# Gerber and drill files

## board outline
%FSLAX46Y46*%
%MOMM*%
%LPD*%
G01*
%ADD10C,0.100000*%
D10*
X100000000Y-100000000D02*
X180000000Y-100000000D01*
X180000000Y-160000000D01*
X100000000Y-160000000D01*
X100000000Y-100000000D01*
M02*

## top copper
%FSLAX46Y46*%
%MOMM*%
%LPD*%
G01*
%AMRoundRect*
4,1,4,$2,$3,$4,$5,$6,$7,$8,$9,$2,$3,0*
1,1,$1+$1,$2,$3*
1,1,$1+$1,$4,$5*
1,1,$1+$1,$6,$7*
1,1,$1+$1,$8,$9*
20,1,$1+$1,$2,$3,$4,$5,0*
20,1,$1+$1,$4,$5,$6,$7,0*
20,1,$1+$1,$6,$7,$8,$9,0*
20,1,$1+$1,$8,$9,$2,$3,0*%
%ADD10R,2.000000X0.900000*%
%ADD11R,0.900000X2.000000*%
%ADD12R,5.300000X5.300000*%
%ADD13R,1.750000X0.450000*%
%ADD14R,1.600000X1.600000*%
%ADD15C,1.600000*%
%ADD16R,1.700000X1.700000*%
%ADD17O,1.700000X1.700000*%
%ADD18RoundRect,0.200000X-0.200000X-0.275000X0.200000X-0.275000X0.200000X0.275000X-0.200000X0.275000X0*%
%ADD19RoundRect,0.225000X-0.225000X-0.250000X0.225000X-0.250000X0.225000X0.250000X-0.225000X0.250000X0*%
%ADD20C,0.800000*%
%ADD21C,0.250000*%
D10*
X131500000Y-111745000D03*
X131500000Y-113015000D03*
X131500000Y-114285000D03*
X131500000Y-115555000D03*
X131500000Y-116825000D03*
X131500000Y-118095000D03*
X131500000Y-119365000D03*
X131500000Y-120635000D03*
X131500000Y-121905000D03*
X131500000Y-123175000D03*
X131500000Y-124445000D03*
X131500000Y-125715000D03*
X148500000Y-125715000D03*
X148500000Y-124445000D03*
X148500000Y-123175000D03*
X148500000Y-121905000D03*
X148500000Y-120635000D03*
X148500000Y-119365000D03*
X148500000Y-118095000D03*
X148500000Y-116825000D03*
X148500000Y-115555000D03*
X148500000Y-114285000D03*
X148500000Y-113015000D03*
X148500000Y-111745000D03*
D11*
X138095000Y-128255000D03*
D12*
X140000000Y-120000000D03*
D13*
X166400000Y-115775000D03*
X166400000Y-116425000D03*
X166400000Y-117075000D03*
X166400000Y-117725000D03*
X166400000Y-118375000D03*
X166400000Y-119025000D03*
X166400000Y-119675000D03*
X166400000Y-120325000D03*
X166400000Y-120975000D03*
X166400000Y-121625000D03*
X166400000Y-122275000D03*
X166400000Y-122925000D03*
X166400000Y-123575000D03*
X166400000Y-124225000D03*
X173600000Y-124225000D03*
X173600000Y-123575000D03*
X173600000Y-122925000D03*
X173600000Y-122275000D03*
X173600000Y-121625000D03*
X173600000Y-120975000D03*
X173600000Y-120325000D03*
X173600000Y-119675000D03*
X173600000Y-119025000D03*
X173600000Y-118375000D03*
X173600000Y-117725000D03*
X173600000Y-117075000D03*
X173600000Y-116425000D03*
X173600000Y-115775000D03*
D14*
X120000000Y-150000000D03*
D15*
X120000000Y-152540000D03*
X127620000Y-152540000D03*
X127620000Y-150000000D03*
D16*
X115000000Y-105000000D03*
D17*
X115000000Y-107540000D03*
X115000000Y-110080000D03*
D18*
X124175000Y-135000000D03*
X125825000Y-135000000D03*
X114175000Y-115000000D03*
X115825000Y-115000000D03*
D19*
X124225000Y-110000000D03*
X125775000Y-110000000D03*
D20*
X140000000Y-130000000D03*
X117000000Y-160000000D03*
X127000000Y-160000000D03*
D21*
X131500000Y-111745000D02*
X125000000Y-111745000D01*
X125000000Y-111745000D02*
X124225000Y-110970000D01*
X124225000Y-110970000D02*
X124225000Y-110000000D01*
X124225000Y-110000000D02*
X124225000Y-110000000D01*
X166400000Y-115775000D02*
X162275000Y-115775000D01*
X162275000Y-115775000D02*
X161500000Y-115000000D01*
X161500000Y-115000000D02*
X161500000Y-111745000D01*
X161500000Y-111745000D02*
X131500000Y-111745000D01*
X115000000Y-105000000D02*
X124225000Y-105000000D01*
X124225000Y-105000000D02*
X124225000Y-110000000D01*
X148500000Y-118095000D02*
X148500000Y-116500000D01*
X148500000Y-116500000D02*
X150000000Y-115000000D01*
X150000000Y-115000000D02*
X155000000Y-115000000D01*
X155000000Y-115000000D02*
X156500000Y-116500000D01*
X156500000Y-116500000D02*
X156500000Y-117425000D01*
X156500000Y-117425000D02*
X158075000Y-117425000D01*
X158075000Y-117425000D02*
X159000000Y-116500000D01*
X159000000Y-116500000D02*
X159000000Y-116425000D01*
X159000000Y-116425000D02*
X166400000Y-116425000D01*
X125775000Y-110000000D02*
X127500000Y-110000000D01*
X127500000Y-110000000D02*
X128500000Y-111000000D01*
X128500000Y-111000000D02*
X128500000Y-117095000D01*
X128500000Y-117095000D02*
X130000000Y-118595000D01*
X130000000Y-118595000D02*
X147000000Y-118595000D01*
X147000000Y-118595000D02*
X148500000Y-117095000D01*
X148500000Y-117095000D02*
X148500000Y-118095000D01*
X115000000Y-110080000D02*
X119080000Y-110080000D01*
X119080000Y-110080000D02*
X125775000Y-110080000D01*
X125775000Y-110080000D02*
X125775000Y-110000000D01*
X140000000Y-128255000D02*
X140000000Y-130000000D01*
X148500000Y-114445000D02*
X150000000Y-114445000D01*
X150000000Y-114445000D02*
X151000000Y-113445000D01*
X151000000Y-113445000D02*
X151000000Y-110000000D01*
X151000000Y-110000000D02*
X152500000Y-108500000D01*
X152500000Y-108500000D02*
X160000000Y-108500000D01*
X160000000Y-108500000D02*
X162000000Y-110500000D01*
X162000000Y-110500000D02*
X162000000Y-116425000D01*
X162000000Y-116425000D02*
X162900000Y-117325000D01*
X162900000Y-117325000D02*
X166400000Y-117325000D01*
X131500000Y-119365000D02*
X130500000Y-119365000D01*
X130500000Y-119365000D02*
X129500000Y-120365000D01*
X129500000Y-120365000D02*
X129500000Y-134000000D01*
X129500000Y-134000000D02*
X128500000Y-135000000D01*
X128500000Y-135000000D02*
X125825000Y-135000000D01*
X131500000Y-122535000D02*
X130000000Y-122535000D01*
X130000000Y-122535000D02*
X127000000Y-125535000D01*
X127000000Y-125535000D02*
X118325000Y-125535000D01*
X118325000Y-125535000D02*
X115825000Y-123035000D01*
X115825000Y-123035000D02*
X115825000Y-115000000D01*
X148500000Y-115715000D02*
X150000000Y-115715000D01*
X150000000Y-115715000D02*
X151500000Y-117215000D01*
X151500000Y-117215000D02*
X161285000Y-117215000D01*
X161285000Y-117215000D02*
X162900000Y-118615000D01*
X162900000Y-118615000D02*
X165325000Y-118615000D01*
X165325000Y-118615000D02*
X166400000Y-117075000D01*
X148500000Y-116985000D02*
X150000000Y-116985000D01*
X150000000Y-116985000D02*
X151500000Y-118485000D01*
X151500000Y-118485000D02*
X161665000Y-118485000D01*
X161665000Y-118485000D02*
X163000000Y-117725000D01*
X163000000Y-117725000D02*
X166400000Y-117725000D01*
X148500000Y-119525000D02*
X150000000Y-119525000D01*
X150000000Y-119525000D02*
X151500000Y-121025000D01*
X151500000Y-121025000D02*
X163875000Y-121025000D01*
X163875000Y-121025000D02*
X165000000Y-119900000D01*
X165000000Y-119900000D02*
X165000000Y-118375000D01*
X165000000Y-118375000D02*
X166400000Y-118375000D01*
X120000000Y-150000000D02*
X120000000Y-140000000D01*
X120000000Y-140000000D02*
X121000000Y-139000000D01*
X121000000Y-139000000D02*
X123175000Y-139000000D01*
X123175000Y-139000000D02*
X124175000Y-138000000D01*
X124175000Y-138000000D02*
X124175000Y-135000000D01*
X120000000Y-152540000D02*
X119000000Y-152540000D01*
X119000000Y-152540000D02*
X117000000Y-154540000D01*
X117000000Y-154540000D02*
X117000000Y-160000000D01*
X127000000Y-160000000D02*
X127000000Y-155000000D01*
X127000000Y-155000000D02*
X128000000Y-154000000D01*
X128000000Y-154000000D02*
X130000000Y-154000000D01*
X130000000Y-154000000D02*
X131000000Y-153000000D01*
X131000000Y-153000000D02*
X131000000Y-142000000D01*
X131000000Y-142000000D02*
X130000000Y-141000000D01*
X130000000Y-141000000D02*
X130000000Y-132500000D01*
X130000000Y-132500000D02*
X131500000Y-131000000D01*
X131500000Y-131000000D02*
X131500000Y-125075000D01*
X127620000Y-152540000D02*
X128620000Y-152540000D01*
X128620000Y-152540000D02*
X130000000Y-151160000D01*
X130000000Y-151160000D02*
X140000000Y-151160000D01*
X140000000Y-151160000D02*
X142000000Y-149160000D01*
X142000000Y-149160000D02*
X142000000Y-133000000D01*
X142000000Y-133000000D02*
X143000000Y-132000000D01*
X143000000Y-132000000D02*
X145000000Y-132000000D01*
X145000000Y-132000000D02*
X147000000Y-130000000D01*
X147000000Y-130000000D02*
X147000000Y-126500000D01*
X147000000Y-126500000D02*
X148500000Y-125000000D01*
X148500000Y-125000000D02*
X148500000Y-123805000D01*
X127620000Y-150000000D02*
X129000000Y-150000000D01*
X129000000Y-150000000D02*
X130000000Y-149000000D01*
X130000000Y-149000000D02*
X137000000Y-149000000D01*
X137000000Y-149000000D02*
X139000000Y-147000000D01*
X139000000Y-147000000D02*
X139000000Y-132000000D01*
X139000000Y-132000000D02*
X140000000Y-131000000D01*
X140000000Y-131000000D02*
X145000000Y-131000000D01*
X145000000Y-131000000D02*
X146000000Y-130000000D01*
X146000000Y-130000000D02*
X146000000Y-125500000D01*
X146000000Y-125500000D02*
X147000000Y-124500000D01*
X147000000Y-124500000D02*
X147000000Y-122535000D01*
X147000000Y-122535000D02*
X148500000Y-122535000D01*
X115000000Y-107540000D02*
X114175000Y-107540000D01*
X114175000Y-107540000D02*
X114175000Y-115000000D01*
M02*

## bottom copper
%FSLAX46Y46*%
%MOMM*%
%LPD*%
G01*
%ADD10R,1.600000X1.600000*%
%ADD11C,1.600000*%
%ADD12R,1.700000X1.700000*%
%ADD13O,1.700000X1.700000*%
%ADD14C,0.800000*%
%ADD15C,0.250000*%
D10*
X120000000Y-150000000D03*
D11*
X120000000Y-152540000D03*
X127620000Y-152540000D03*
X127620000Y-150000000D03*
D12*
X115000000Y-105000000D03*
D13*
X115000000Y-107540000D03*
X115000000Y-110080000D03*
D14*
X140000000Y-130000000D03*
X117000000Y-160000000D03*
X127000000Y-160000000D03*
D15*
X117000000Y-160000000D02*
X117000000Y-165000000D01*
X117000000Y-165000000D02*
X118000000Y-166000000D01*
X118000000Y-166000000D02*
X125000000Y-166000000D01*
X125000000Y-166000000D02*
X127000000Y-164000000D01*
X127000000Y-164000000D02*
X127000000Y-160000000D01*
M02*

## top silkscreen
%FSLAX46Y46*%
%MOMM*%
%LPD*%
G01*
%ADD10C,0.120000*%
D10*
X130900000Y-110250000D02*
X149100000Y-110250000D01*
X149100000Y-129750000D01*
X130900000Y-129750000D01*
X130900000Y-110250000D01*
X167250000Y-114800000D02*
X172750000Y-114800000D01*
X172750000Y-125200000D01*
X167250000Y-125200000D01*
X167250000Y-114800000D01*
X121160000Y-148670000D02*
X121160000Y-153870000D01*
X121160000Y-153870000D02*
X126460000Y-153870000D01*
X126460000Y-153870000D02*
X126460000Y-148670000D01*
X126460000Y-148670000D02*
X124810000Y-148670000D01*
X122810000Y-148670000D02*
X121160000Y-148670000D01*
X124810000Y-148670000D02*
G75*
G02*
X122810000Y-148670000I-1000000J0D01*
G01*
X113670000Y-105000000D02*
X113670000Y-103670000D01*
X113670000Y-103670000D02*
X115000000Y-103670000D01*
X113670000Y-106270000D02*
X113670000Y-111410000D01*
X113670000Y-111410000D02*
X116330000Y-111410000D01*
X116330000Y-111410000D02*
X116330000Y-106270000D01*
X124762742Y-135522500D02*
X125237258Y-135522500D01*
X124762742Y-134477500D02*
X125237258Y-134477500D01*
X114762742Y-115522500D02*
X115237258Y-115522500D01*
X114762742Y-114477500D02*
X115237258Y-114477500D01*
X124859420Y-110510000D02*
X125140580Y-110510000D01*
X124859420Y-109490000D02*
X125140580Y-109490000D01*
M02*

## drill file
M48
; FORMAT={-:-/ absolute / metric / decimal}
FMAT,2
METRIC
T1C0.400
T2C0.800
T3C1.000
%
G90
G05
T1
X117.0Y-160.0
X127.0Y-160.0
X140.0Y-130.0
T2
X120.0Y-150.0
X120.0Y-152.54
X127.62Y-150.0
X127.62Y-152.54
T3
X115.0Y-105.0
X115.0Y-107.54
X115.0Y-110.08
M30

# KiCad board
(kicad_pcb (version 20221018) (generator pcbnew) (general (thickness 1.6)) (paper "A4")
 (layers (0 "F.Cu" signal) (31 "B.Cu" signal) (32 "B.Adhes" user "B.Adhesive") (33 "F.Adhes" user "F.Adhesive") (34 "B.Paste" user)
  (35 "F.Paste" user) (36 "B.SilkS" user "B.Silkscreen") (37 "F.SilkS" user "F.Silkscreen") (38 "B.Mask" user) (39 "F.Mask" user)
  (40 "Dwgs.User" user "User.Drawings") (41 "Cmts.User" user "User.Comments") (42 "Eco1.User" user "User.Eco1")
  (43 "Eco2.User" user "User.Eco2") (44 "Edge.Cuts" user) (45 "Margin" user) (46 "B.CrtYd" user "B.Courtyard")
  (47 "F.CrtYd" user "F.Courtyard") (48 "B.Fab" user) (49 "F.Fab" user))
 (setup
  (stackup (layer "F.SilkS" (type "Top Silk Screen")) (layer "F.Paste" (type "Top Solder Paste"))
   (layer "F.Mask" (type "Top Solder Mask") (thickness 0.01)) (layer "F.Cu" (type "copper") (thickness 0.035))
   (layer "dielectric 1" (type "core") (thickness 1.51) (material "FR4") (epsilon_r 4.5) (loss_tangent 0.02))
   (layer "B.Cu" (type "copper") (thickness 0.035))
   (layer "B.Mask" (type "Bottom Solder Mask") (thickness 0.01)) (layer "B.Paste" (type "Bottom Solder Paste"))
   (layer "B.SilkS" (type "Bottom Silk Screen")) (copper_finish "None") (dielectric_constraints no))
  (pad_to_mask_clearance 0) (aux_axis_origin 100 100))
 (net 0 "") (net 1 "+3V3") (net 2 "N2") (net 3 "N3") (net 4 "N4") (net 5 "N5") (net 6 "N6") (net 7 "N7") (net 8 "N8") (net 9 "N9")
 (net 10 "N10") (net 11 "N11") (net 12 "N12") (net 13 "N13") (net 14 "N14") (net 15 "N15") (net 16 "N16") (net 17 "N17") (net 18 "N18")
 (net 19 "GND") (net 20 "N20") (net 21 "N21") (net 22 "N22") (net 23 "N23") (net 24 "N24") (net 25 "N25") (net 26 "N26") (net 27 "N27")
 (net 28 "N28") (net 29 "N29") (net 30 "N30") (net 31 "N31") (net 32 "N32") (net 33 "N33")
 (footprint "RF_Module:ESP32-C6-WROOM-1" (layer "F.Cu") (at 140 120 0)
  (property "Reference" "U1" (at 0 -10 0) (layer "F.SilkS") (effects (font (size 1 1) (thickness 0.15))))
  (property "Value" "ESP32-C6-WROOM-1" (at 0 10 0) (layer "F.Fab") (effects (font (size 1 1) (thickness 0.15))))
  (fp_rect (start -9.1 -9.75) (end 9.1 9.75) (layer "F.SilkS") (width 0.12) (fill none))
  (pad "1" smd rect (at -8.5 -8.255) (size 2 0.9) (layers "F.Cu" "F.Paste" "F.Mask") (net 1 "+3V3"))
  (pad "2" smd rect (at -8.5 -6.985) (size 2 0.9) (layers "F.Cu" "F.Paste" "F.Mask") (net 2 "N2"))
  (pad "3" smd rect (at -8.5 -5.715) (size 2 0.9) (layers "F.Cu" "F.Paste" "F.Mask") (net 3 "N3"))
  (pad "4" smd rect (at -8.5 -4.445) (size 2 0.9) (layers "F.Cu" "F.Paste" "F.Mask") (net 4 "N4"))
  (pad "5" smd rect (at -8.5 -3.175) (size 2 0.9) (layers "F.Cu" "F.Paste" "F.Mask") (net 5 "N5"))
  (pad "6" smd rect (at -8.5 -1.905) (size 2 0.9) (layers "F.Cu" "F.Paste" "F.Mask") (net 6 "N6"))
  (pad "7" smd rect (at -8.5 -0.635) (size 2 0.9) (layers "F.Cu" "F.Paste" "F.Mask") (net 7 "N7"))
  (pad "8" smd rect (at -8.5 0.635) (size 2 0.9) (layers "F.Cu" "F.Paste" "F.Mask") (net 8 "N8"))
  (pad "9" smd rect (at -8.5 1.905) (size 2 0.9) (layers "F.Cu" "F.Paste" "F.Mask") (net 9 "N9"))
  (pad "10" smd rect (at -8.5 3.175) (size 2 0.9) (layers "F.Cu" "F.Paste" "F.Mask") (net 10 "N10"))
  (pad "11" smd rect (at -8.5 4.445) (size 2 0.9) (layers "F.Cu" "F.Paste" "F.Mask") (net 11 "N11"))
  (pad "12" smd rect (at -8.5 5.715) (size 2 0.9) (layers "F.Cu" "F.Paste" "F.Mask") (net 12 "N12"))
  (pad "13" smd rect (at 8.5 5.715) (size 2 0.9) (layers "F.Cu" "F.Paste" "F.Mask") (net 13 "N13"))
  (pad "14" smd rect (at 8.5 4.445) (size 2 0.9) (layers "F.Cu" "F.Paste" "F.Mask") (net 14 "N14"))
  (pad "15" smd rect (at 8.5 3.175) (size 2 0.9) (layers "F.Cu" "F.Paste" "F.Mask") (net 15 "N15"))
  (pad "16" smd rect (at 8.5 1.905) (size 2 0.9) (layers "F.Cu" "F.Paste" "F.Mask") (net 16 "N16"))
  (pad "17" smd rect (at 8.5 0.635) (size 2 0.9) (layers "F.Cu" "F.Paste" "F.Mask") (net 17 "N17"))
  (pad "18" smd rect (at 8.5 -0.635) (size 2 0.9) (layers "F.Cu" "F.Paste" "F.Mask") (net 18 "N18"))
  (pad "19" smd rect (at 8.5 -1.905) (size 2 0.9) (layers "F.Cu" "F.Paste" "F.Mask") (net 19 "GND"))
  (pad "20" smd rect (at 8.5 -3.175) (size 2 0.9) (layers "F.Cu" "F.Paste" "F.Mask") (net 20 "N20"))
  (pad "21" smd rect (at 8.5 -4.445) (size 2 0.9) (layers "F.Cu" "F.Paste" "F.Mask") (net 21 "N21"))
  (pad "22" smd rect (at 8.5 -5.715) (size 2 0.9) (layers "F.Cu" "F.Paste" "F.Mask") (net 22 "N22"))
  (pad "23" smd rect (at 8.5 -6.985) (size 2 0.9) (layers "F.Cu" "F.Paste" "F.Mask") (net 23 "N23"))
  (pad "24" smd rect (at 8.5 -8.255) (size 2 0.9) (layers "F.Cu" "F.Paste" "F.Mask") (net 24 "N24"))
  (pad "25" smd rect (at -1.905 8.255 90) (size 2 0.9) (layers "F.Cu" "F.Paste" "F.Mask") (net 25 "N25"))
  (pad "39" smd rect (at 0 0) (size 5.3 5.3) (layers "F.Cu" "F.Paste" "F.Mask") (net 19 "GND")))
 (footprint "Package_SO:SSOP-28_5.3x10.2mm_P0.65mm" (layer "F.Cu") (at 170 120 0)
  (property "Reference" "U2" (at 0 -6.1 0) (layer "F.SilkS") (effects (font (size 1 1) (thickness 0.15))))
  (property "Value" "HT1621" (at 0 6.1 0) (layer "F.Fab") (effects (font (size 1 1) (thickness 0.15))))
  (fp_rect (start -2.75 -5.2) (end 2.75 5.2) (layer "F.SilkS") (width 0.12) (fill none))
  (pad "1" smd rect (at -3.6 -4.225) (size 1.75 0.45) (layers "F.Cu" "F.Paste" "F.Mask") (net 1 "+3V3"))
  (pad "2" smd rect (at -3.6 -3.575) (size 1.75 0.45) (layers "F.Cu" "F.Paste" "F.Mask") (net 19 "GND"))
  (pad "3" smd rect (at -3.6 -2.925) (size 1.75 0.45) (layers "F.Cu" "F.Paste" "F.Mask") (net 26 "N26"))
  (pad "4" smd rect (at -3.6 -2.275) (size 1.75 0.45) (layers "F.Cu" "F.Paste" "F.Mask") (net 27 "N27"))
  (pad "5" smd rect (at -3.6 -1.625) (size 1.75 0.45) (layers "F.Cu" "F.Paste" "F.Mask") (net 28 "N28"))
  (pad "6" smd rect (at -3.6 -0.975) (size 1.75 0.45) (layers "F.Cu" "F.Paste" "F.Mask"))
  (pad "7" smd rect (at -3.6 -0.325) (size 1.75 0.45) (layers "F.Cu" "F.Paste" "F.Mask"))
  (pad "8" smd rect (at -3.6 0.325) (size 1.75 0.45) (layers "F.Cu" "F.Paste" "F.Mask"))
  (pad "9" smd rect (at -3.6 0.975) (size 1.75 0.45) (layers "F.Cu" "F.Paste" "F.Mask"))
  (pad "10" smd rect (at -3.6 1.625) (size 1.75 0.45) (layers "F.Cu" "F.Paste" "F.Mask"))
  (pad "11" smd rect (at -3.6 2.275) (size 1.75 0.45) (layers "F.Cu" "F.Paste" "F.Mask"))
  (pad "12" smd rect (at -3.6 2.925) (size 1.75 0.45) (layers "F.Cu" "F.Paste" "F.Mask"))
  (pad "13" smd rect (at -3.6 3.575) (size 1.75 0.45) (layers "F.Cu" "F.Paste" "F.Mask"))
  (pad "14" smd rect (at -3.6 4.225) (size 1.75 0.45) (layers "F.Cu" "F.Paste" "F.Mask"))
  (pad "15" smd rect (at 3.6 4.225) (size 1.75 0.45) (layers "F.Cu" "F.Paste" "F.Mask"))
  (pad "16" smd rect (at 3.6 3.575) (size 1.75 0.45) (layers "F.Cu" "F.Paste" "F.Mask"))
  (pad "17" smd rect (at 3.6 2.925) (size 1.75 0.45) (layers "F.Cu" "F.Paste" "F.Mask"))
  (pad "18" smd rect (at 3.6 2.275) (size 1.75 0.45) (layers "F.Cu" "F.Paste" "F.Mask"))
  (pad "19" smd rect (at 3.6 1.625) (size 1.75 0.45) (layers "F.Cu" "F.Paste" "F.Mask"))
  (pad "20" smd rect (at 3.6 0.975) (size 1.75 0.45) (layers "F.Cu" "F.Paste" "F.Mask"))
  (pad "21" smd rect (at 3.6 0.325) (size 1.75 0.45) (layers "F.Cu" "F.Paste" "F.Mask"))
  (pad "22" smd rect (at 3.6 -0.325) (size 1.75 0.45) (layers "F.Cu" "F.Paste" "F.Mask"))
  (pad "23" smd rect (at 3.6 -0.975) (size 1.75 0.45) (layers "F.Cu" "F.Paste" "F.Mask"))
  (pad "24" smd rect (at 3.6 -1.625) (size 1.75 0.45) (layers "F.Cu" "F.Paste" "F.Mask"))
  (pad "25" smd rect (at 3.6 -2.275) (size 1.75 0.45) (layers "F.Cu" "F.Paste" "F.Mask"))
  (pad "26" smd rect (at 3.6 -2.925) (size 1.75 0.45) (layers "F.Cu" "F.Paste" "F.Mask"))
  (pad "27" smd rect (at 3.6 -3.575) (size 1.75 0.45) (layers "F.Cu" "F.Paste" "F.Mask"))
  (pad "28" smd rect (at 3.6 -4.225) (size 1.75 0.45) (layers "F.Cu" "F.Paste" "F.Mask")))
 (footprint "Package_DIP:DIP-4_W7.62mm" (layer "F.Cu") (at 120 150 0)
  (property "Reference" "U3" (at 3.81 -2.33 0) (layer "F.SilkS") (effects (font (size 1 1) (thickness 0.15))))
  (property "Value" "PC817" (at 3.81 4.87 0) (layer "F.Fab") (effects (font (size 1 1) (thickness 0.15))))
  (fp_line (start 1.16 -1.33) (end 1.16 3.87) (layer "F.SilkS") (width 0.12))
  (fp_line (start 1.16 3.87) (end 6.46 3.87) (layer "F.SilkS") (width 0.12))
  (fp_line (start 6.46 3.87) (end 6.46 -1.33) (layer "F.SilkS") (width 0.12))
  (fp_line (start 6.46 -1.33) (end 4.81 -1.33) (layer "F.SilkS") (width 0.12))
  (fp_line (start 2.81 -1.33) (end 1.16 -1.33) (layer "F.SilkS") (width 0.12))
  (fp_arc (start 4.81 -1.33) (mid 3.81 -0.33) (end 2.81 -1.33) (layer "F.SilkS") (width 0.12))
  (pad "1" thru_hole rect (at 0 0) (size 1.6 1.6) (drill 0.8) (layers *.Cu *.Mask) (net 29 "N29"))
  (pad "2" thru_hole circle (at 0 2.54) (size 1.6 1.6) (drill 0.8) (layers *.Cu *.Mask) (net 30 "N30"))
  (pad "3" thru_hole circle (at 7.62 2.54) (size 1.6 1.6) (drill 0.8) (layers *.Cu *.Mask) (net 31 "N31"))
  (pad "4" thru_hole circle (at 7.62 0) (size 1.6 1.6) (drill 0.8) (layers *.Cu *.Mask) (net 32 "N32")))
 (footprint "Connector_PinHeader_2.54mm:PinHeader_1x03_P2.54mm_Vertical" (layer "F.Cu") (at 115 105 0)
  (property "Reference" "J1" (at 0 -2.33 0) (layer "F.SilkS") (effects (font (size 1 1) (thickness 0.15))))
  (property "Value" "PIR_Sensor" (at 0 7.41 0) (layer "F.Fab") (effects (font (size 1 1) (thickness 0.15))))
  (fp_line (start -1.33 0) (end -1.33 -1.33) (layer "F.SilkS") (width 0.12))
  (fp_line (start -1.33 -1.33) (end 0 -1.33) (layer "F.SilkS") (width 0.12))
  (fp_line (start -1.33 1.27) (end -1.33 6.41) (layer "F.SilkS") (width 0.12))
  (fp_line (start -1.33 6.41) (end 1.33 6.41) (layer "F.SilkS") (width 0.12))
  (fp_line (start 1.33 6.41) (end 1.33 1.27) (layer "F.SilkS") (width 0.12))
  (pad "1" thru_hole rect (at 0 0) (size 1.7 1.7) (drill 1) (layers *.Cu *.Mask) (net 1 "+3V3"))
  (pad "2" thru_hole oval (at 0 2.54) (size 1.7 1.7) (drill 1) (layers *.Cu *.Mask) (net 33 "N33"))
  (pad "3" thru_hole oval (at 0 5.08) (size 1.7 1.7) (drill 1) (layers *.Cu *.Mask) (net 19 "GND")))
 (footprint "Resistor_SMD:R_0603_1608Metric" (layer "F.Cu") (at 125 135 0)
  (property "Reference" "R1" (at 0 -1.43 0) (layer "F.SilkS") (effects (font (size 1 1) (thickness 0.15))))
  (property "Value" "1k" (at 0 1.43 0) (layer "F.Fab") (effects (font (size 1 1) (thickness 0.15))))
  (fp_line (start -0.237258 0.5225) (end 0.237258 0.5225) (layer "F.SilkS") (width 0.12))
  (fp_line (start -0.237258 -0.5225) (end 0.237258 -0.5225) (layer "F.SilkS") (width 0.12))
  (pad "1" smd roundrect (at -0.825 0) (size 0.8 0.95) (layers "F.Cu" "F.Paste" "F.Mask") (roundrect_rratio 0.25) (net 29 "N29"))
  (pad "2" smd roundrect (at 0.825 0) (size 0.8 0.95) (layers "F.Cu" "F.Paste" "F.Mask") (roundrect_rratio 0.25) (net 7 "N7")))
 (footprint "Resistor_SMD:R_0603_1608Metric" (layer "F.Cu") (at 115 115 0)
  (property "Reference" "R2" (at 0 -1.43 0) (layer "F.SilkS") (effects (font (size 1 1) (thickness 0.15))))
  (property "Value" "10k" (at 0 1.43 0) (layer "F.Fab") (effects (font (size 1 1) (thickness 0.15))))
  (fp_line (start -0.237258 0.5225) (end 0.237258 0.5225) (layer "F.SilkS") (width 0.12))
  (fp_line (start -0.237258 -0.5225) (end 0.237258 -0.5225) (layer "F.SilkS") (width 0.12))
  (pad "1" smd roundrect (at -0.825 0) (size 0.8 0.95) (layers "F.Cu" "F.Paste" "F.Mask") (roundrect_rratio 0.25) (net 33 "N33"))
  (pad "2" smd roundrect (at 0.825 0) (size 0.8 0.95) (layers "F.Cu" "F.Paste" "F.Mask") (roundrect_rratio 0.25) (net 9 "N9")))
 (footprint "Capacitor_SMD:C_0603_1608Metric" (layer "F.Cu") (at 125 110 0)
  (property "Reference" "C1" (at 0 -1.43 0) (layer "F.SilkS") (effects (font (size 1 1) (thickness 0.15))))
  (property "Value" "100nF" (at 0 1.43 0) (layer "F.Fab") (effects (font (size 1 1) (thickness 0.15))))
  (fp_line (start -0.14058 0.51) (end 0.14058 0.51) (layer "F.SilkS") (width 0.12))
  (fp_line (start -0.14058 -0.51) (end 0.14058 -0.51) (layer "F.SilkS") (width 0.12))
  (pad "1" smd roundrect (at -0.775 0) (size 0.9 0.95) (layers "F.Cu" "F.Paste" "F.Mask") (roundrect_rratio 0.25) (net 1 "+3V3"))
  (pad "2" smd roundrect (at 0.775 0) (size 0.9 0.95) (layers "F.Cu" "F.Paste" "F.Mask") (roundrect_rratio 0.25) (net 19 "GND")))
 (gr_rect (start 100 100) (end 180 160) (layer "Edge.Cuts") (width 0.1) (fill none))
 (segment (start 131.5 111.745) (end 125 111.745) (width 0.25) (layer "F.Cu") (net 1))
 (segment (start 125 111.745) (end 124.225 110.97) (width 0.25) (layer "F.Cu") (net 1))
 (segment (start 124.225 110.97) (end 124.225 110) (width 0.25) (layer "F.Cu") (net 1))
 (segment (start 124.225 110) (end 124.225 110) (width 0.25) (layer "F.Cu") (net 1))
 (segment (start 166.4 115.775) (end 162.275 115.775) (width 0.25) (layer "F.Cu") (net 1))
 (segment (start 162.275 115.775) (end 161.5 115) (width 0.25) (layer "F.Cu") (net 1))
 (segment (start 161.5 115) (end 161.5 111.745) (width 0.25) (layer "F.Cu") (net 1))
 (segment (start 161.5 111.745) (end 131.5 111.745) (width 0.25) (layer "F.Cu") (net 1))
 (segment (start 115 105) (end 124.225 105) (width 0.25) (layer "F.Cu") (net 1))
 (segment (start 124.225 105) (end 124.225 110) (width 0.25) (layer "F.Cu") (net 1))
 (segment (start 148.5 118.095) (end 148.5 116.5) (width 0.25) (layer "F.Cu") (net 19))
 (segment (start 148.5 116.5) (end 150 115) (width 0.25) (layer "F.Cu") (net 19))
 (segment (start 150 115) (end 155 115) (width 0.25) (layer "F.Cu") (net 19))
 (segment (start 155 115) (end 156.5 116.5) (width 0.25) (layer "F.Cu") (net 19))
 (segment (start 156.5 116.5) (end 156.5 117.425) (width 0.25) (layer "F.Cu") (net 19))
 (segment (start 156.5 117.425) (end 158.075 117.425) (width 0.25) (layer "F.Cu") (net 19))
 (segment (start 158.075 117.425) (end 159 116.5) (width 0.25) (layer "F.Cu") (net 19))
 (segment (start 159 116.5) (end 159 116.425) (width 0.25) (layer "F.Cu") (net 19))
 (segment (start 159 116.425) (end 166.4 116.425) (width 0.25) (layer "F.Cu") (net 19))
 (segment (start 125.775 110) (end 127.5 110) (width 0.25) (layer "F.Cu") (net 19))
 (segment (start 127.5 110) (end 128.5 111) (width 0.25) (layer "F.Cu") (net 19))
 (segment (start 128.5 111) (end 128.5 117.095) (width 0.25) (layer "F.Cu") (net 19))
 (segment (start 128.5 117.095) (end 130 118.595) (width 0.25) (layer "F.Cu") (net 19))
 (segment (start 130 118.595) (end 147 118.595) (width 0.25) (layer "F.Cu") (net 19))
 (segment (start 147 118.595) (end 148.5 117.095) (width 0.25) (layer "F.Cu") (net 19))
 (segment (start 148.5 117.095) (end 148.5 118.095) (width 0.25) (layer "F.Cu") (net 19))
 (segment (start 115 110.08) (end 119.08 110.08) (width 0.25) (layer "F.Cu") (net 19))
 (segment (start 119.08 110.08) (end 125.775 110.08) (width 0.25) (layer "F.Cu") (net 19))
 (segment (start 125.775 110.08) (end 125.775 110) (width 0.25) (layer "F.Cu") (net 19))
 (segment (start 140 128.255) (end 140 130) (width 0.25) (layer "F.Cu") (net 19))
 (via (at 140 130) (size 0.8) (drill 0.4) (layers "F.Cu" "B.Cu") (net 19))
 (segment (start 148.5 114.445) (end 150 114.445) (width 0.25) (layer "F.Cu") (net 3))
 (segment (start 150 114.445) (end 151 113.445) (width 0.25) (layer "F.Cu") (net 3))
 (segment (start 151 113.445) (end 151 110) (width 0.25) (layer "F.Cu") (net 3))
 (segment (start 151 110) (end 152.5 108.5) (width 0.25) (layer "F.Cu") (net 3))
 (segment (start 152.5 108.5) (end 160 108.5) (width 0.25) (layer "F.Cu") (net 3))
 (segment (start 160 108.5) (end 162 110.5) (width 0.25) (layer "F.Cu") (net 3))
 (segment (start 162 110.5) (end 162 116.425) (width 0.25) (layer "F.Cu") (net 3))
 (segment (start 162 116.425) (end 162.9 117.325) (width 0.25) (layer "F.Cu") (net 3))
 (segment (start 162.9 117.325) (end 166.4 117.325) (width 0.25) (layer "F.Cu") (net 3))
 (segment (start 131.5 119.365) (end 130.5 119.365) (width 0.25) (layer "F.Cu") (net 7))
 (segment (start 130.5 119.365) (end 129.5 120.365) (width 0.25) (layer "F.Cu") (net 7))
 (segment (start 129.5 120.365) (end 129.5 134) (width 0.25) (layer "F.Cu") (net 7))
 (segment (start 129.5 134) (end 128.5 135) (width 0.25) (layer "F.Cu") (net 7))
 (segment (start 128.5 135) (end 125.825 135) (width 0.25) (layer "F.Cu") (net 7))
 (segment (start 131.5 122.535) (end 130 122.535) (width 0.25) (layer "F.Cu") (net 9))
 (segment (start 130 122.535) (end 127 125.535) (width 0.25) (layer "F.Cu") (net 9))
 (segment (start 127 125.535) (end 118.325 125.535) (width 0.25) (layer "F.Cu") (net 9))
 (segment (start 118.325 125.535) (end 115.825 123.035) (width 0.25) (layer "F.Cu") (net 9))
 (segment (start 115.825 123.035) (end 115.825 115) (width 0.25) (layer "F.Cu") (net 9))
 (segment (start 148.5 115.715) (end 150 115.715) (width 0.25) (layer "F.Cu") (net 26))
 (segment (start 150 115.715) (end 151.5 117.215) (width 0.25) (layer "F.Cu") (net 26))
 (segment (start 151.5 117.215) (end 161.285 117.215) (width 0.25) (layer "F.Cu") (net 26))
 (segment (start 161.285 117.215) (end 162.9 118.615) (width 0.25) (layer "F.Cu") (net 26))
 (segment (start 162.9 118.615) (end 165.325 118.615) (width 0.25) (layer "F.Cu") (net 26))
 (segment (start 165.325 118.615) (end 166.4 117.075) (width 0.25) (layer "F.Cu") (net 26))
 (segment (start 148.5 116.985) (end 150 116.985) (width 0.25) (layer "F.Cu") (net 27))
 (segment (start 150 116.985) (end 151.5 118.485) (width 0.25) (layer "F.Cu") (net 27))
 (segment (start 151.5 118.485) (end 161.665 118.485) (width 0.25) (layer "F.Cu") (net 27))
 (segment (start 161.665 118.485) (end 163 117.725) (width 0.25) (layer "F.Cu") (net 27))
 (segment (start 163 117.725) (end 166.4 117.725) (width 0.25) (layer "F.Cu") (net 27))
 (segment (start 148.5 119.525) (end 150 119.525) (width 0.25) (layer "F.Cu") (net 28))
 (segment (start 150 119.525) (end 151.5 121.025) (width 0.25) (layer "F.Cu") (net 28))
 (segment (start 151.5 121.025) (end 163.875 121.025) (width 0.25) (layer "F.Cu") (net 28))
 (segment (start 163.875 121.025) (end 165 119.9) (width 0.25) (layer "F.Cu") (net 28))
 (segment (start 165 119.9) (end 165 118.375) (width 0.25) (layer "F.Cu") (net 28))
 (segment (start 165 118.375) (end 166.4 118.375) (width 0.25) (layer "F.Cu") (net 28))
 (segment (start 120 150) (end 120 140) (width 0.25) (layer "F.Cu") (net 29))
 (segment (start 120 140) (end 121 139) (width 0.25) (layer "F.Cu") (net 29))
 (segment (start 121 139) (end 123.175 139) (width 0.25) (layer "F.Cu") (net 29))
 (segment (start 123.175 139) (end 124.175 138) (width 0.25) (layer "F.Cu") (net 29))
 (segment (start 124.175 138) (end 124.175 135) (width 0.25) (layer "F.Cu") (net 29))
 (segment (start 120 152.54) (end 119 152.54) (width 0.25) (layer "F.Cu") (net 30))
 (segment (start 119 152.54) (end 117 154.54) (width 0.25) (layer "F.Cu") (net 30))
 (segment (start 117 154.54) (end 117 160) (width 0.25) (layer "F.Cu") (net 30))
 (via (at 117 160) (size 0.8) (drill 0.4) (layers "F.Cu" "B.Cu") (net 30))
 (segment (start 117 160) (end 117 165) (width 0.25) (layer "B.Cu") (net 30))
 (segment (start 117 165) (end 118 166) (width 0.25) (layer "B.Cu") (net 30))
 (segment (start 118 166) (end 125 166) (width 0.25) (layer "B.Cu") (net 30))
 (segment (start 125 166) (end 127 164) (width 0.25) (layer "B.Cu") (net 30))
 (segment (start 127 164) (end 127 160) (width 0.25) (layer "B.Cu") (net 30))
 (via (at 127 160) (size 0.8) (drill 0.4) (layers "F.Cu" "B.Cu") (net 30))
 (segment (start 127 160) (end 127 155) (width 0.25) (layer "F.Cu") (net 30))
 (segment (start 127 155) (end 128 154) (width 0.25) (layer "F.Cu") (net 30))
 (segment (start 128 154) (end 130 154) (width 0.25) (layer "F.Cu") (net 30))
 (segment (start 130 154) (end 131 153) (width 0.25) (layer "F.Cu") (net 30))
 (segment (start 131 153) (end 131 142) (width 0.25) (layer "F.Cu") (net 30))
 (segment (start 131 142) (end 130 141) (width 0.25) (layer "F.Cu") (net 30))
 (segment (start 130 141) (end 130 132.5) (width 0.25) (layer "F.Cu") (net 30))
 (segment (start 130 132.5) (end 131.5 131) (width 0.25) (layer "F.Cu") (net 30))
 (segment (start 131.5 131) (end 131.5 125.075) (width 0.25) (layer "F.Cu") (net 30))
 (segment (start 127.62 152.54) (end 128.62 152.54) (width 0.25) (layer "F.Cu") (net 31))
 (segment (start 128.62 152.54) (end 130 151.16) (width 0.25) (layer "F.Cu") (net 31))
 (segment (start 130 151.16) (end 140 151.16) (width 0.25) (layer "F.Cu") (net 31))
 (segment (start 140 151.16) (end 142 149.16) (width 0.25) (layer "F.Cu") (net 31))
 (segment (start 142 149.16) (end 142 133) (width 0.25) (layer "F.Cu") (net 31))
 (segment (start 142 133) (end 143 132) (width 0.25) (layer "F.Cu") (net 31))
 (segment (start 143 132) (end 145 132) (width 0.25) (layer "F.Cu") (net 31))
 (segment (start 145 132) (end 147 130) (width 0.25) (layer "F.Cu") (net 31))
 (segment (start 147 130) (end 147 126.5) (width 0.25) (layer "F.Cu") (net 31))
 (segment (start 147 126.5) (end 148.5 125) (width 0.25) (layer "F.Cu") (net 31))
 (segment (start 148.5 125) (end 148.5 123.805) (width 0.25) (layer "F.Cu") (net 31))
 (segment (start 127.62 150) (end 129 150) (width 0.25) (layer "F.Cu") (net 32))
 (segment (start 129 150) (end 130 149) (width 0.25) (layer "F.Cu") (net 32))
 (segment (start 130 149) (end 137 149) (width 0.25) (layer "F.Cu") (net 32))
 (segment (start 137 149) (end 139 147) (width 0.25) (layer "F.Cu") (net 32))
 (segment (start 139 147) (end 139 132) (width 0.25) (layer "F.Cu") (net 32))
 (segment (start 139 132) (end 140 131) (width 0.25) (layer "F.Cu") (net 32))
 (segment (start 140 131) (end 145 131) (width 0.25) (layer "F.Cu") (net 32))
 (segment (start 145 131) (end 146 130) (width 0.25) (layer "F.Cu") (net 32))
 (segment (start 146 130) (end 146 125.5) (width 0.25) (layer "F.Cu") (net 32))
 (segment (start 146 125.5) (end 147 124.5) (width 0.25) (layer "F.Cu") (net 32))
 (segment (start 147 124.5) (end 147 122.535) (width 0.25) (layer "F.Cu") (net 32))
 (segment (start 147 122.535) (end 148.5 122.535) (width 0.25) (layer "F.Cu") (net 32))
 (segment (start 115 107.54) (end 114.175 107.54) (width 0.25) (layer "F.Cu") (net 33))
 (segment (start 114.175 107.54) (end 114.175 115) (width 0.25) (layer "F.Cu") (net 33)))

